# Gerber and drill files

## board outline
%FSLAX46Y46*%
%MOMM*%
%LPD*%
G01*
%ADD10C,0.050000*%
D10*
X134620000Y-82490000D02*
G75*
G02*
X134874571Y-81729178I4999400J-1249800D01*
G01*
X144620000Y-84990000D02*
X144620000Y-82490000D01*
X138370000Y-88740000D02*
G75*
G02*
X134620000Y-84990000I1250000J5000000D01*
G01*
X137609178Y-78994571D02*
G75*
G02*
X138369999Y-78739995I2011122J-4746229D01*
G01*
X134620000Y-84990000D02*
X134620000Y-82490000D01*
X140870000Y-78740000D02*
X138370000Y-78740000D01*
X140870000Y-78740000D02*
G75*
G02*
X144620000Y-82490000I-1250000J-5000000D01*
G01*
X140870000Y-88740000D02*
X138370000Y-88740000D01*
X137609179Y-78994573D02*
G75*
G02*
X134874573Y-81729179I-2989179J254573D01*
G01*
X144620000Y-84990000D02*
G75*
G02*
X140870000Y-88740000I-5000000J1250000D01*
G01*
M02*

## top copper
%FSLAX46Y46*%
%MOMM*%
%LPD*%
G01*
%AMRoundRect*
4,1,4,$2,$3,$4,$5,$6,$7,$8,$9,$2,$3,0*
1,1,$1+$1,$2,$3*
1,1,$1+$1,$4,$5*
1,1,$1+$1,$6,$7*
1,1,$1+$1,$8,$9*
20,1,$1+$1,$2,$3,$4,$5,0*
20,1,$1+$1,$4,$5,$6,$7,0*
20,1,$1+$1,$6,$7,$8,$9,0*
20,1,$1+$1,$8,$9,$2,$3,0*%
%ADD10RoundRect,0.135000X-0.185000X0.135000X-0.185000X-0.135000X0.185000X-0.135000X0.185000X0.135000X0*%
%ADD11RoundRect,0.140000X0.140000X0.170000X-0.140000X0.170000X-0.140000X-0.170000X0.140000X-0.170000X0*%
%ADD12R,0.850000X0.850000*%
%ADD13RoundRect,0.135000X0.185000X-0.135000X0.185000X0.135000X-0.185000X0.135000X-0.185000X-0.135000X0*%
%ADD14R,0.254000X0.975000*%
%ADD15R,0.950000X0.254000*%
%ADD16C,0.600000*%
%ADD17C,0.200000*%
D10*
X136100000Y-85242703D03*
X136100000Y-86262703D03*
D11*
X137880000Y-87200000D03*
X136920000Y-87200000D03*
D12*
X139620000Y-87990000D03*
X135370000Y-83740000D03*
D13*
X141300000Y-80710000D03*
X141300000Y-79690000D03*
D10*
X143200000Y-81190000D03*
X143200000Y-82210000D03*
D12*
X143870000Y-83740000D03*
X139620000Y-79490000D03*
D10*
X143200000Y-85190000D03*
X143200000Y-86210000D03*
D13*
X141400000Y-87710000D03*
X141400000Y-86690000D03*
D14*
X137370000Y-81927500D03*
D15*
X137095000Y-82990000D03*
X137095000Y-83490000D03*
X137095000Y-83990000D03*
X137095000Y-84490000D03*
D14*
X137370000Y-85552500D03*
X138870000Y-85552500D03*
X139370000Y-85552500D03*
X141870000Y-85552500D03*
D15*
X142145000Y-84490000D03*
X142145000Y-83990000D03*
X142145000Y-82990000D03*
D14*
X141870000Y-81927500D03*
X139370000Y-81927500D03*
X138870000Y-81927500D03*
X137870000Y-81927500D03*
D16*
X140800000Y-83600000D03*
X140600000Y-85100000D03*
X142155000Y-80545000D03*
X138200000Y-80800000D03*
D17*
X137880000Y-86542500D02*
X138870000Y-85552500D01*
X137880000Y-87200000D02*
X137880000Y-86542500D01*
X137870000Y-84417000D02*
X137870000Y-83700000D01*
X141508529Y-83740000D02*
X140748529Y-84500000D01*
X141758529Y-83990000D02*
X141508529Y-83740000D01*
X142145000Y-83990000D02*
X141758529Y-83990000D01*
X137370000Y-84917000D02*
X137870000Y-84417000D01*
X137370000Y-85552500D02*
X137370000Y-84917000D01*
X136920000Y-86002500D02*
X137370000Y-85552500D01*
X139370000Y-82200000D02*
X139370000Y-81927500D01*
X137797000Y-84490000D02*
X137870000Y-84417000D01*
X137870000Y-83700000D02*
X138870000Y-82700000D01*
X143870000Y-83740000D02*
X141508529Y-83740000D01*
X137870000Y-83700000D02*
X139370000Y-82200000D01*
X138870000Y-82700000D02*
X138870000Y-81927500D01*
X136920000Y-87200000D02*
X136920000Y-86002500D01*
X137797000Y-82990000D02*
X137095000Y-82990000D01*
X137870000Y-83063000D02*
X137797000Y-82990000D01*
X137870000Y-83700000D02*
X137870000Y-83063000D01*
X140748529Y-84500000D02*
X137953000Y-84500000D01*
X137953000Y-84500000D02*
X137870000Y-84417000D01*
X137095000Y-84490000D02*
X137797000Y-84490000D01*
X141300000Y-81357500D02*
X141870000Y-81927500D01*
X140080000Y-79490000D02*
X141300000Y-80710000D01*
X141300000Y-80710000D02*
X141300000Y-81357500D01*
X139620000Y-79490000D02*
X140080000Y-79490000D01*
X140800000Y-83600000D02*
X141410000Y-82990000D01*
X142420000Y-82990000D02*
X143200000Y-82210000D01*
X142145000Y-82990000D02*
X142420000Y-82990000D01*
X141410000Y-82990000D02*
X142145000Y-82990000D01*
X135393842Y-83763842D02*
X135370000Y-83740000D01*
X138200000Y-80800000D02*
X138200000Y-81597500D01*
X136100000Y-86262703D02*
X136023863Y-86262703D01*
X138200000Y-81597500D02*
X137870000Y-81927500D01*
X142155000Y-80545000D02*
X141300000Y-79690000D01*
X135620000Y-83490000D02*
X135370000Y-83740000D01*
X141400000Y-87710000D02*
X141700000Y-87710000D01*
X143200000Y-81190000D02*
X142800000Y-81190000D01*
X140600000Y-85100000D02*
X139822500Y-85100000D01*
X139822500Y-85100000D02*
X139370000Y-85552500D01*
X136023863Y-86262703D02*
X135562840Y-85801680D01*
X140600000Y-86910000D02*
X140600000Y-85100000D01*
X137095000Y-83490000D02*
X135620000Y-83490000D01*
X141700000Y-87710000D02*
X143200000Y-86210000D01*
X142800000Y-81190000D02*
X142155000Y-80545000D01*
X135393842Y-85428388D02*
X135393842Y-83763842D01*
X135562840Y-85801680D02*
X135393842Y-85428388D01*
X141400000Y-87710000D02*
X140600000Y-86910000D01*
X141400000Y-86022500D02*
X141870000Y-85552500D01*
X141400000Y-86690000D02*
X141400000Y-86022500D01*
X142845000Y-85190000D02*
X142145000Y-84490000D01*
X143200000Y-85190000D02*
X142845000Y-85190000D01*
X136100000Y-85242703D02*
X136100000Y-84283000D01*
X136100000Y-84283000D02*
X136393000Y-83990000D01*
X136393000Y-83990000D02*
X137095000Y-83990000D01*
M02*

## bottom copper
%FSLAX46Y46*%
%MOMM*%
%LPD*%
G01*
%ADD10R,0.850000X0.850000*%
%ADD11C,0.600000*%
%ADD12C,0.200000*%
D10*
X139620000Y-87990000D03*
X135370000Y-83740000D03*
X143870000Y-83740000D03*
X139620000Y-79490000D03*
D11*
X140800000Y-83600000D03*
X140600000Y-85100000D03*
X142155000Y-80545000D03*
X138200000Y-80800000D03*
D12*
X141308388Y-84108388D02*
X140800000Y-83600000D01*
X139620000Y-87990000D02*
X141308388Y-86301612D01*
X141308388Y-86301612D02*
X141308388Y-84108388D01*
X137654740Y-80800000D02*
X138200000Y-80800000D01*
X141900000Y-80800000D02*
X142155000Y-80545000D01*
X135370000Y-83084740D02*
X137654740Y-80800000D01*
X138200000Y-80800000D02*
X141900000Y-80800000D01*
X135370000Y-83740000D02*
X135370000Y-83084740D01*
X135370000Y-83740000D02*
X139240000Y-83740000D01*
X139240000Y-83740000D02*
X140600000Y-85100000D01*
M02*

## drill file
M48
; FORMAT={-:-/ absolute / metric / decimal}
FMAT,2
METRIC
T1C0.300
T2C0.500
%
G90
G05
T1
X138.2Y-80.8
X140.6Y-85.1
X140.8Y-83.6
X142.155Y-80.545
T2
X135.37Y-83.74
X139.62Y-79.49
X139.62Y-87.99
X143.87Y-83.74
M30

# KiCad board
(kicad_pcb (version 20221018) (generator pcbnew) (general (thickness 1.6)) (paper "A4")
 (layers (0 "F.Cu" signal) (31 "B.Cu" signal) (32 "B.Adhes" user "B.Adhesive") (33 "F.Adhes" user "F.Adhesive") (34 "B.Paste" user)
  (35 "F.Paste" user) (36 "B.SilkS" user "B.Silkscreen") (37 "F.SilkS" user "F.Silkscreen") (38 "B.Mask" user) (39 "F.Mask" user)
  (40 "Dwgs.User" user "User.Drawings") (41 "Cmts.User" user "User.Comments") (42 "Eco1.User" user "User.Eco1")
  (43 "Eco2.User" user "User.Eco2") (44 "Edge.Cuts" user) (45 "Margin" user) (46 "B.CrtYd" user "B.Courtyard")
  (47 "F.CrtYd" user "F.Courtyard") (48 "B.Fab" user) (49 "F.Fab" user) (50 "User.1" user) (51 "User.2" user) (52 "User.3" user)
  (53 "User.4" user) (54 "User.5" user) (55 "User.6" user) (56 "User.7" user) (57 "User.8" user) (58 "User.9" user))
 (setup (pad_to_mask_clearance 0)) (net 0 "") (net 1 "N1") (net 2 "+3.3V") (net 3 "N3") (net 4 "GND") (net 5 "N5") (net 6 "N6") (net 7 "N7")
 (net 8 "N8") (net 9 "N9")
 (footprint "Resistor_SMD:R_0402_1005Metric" (layer "F.Cu") (at 136.1 85.752703 -90)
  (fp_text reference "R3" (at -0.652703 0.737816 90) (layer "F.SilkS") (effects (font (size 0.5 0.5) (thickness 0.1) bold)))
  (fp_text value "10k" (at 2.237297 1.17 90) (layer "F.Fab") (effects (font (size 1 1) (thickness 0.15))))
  (pad "1" smd roundrect (at -0.51 0 270) (size 0.54 0.64) (layers "F.Cu" "F.Paste" "F.Mask") (roundrect_rratio 0.25) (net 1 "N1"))
  (pad "2" smd roundrect (at 0.51 0 270) (size 0.54 0.64) (layers "F.Cu" "F.Paste" "F.Mask") (roundrect_rratio 0.25) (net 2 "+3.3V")))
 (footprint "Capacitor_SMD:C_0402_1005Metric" (layer "F.Cu") (at 137.4 87.2 180)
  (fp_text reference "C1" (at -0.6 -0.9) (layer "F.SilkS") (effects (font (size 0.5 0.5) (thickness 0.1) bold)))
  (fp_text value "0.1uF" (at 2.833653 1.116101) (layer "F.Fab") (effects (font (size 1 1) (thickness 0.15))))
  (pad "1" smd roundrect (at -0.48 0 180) (size 0.56 0.62) (layers "F.Cu" "F.Paste" "F.Mask") (roundrect_rratio 0.25) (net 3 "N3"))
  (pad "2" smd roundrect (at 0.48 0 180) (size 0.56 0.62) (layers "F.Cu" "F.Paste" "F.Mask") (roundrect_rratio 0.25) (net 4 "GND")))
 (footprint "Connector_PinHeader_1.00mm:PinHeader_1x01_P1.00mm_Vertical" (layer "F.Cu") (at 139.62 87.99)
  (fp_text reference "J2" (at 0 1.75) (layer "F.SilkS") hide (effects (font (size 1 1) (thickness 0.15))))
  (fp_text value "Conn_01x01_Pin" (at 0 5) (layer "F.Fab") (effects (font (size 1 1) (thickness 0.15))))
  (pad "1" thru_hole rect (at 0 0) (size 0.85 0.85) (drill 0.5) (layers "*.Cu" "*.Mask") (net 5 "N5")))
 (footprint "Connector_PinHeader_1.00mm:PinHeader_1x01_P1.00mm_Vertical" (layer "F.Cu") (at 135.37 83.74)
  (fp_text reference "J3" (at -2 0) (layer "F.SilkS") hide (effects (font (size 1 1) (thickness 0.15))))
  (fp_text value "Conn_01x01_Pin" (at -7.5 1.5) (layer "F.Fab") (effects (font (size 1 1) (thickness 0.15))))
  (pad "1" thru_hole rect (at 0 0) (size 0.85 0.85) (drill 0.5) (layers "*.Cu" "*.Mask") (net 2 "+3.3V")))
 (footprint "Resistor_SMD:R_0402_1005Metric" (layer "F.Cu") (at 141.3 80.2 90)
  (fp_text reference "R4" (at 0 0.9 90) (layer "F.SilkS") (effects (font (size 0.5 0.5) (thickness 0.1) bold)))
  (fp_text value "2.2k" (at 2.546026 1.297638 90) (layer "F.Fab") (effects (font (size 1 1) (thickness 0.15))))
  (pad "1" smd roundrect (at -0.51 0 90) (size 0.54 0.64) (layers "F.Cu" "F.Paste" "F.Mask") (roundrect_rratio 0.25) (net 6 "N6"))
  (pad "2" smd roundrect (at 0.51 0 90) (size 0.54 0.64) (layers "F.Cu" "F.Paste" "F.Mask") (roundrect_rratio 0.25) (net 2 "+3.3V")))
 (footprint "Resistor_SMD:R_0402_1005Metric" (layer "F.Cu") (at 143.2 81.7 -90)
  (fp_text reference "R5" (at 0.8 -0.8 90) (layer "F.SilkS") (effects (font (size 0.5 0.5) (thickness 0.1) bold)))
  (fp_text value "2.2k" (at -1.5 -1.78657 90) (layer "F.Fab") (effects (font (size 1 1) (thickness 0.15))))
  (pad "1" smd roundrect (at -0.51 0 270) (size 0.54 0.64) (layers "F.Cu" "F.Paste" "F.Mask") (roundrect_rratio 0.25) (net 2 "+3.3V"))
  (pad "2" smd roundrect (at 0.51 0 270) (size 0.54 0.64) (layers "F.Cu" "F.Paste" "F.Mask") (roundrect_rratio 0.25) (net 5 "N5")))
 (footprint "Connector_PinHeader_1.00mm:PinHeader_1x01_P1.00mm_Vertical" (layer "F.Cu") (at 143.87 83.74)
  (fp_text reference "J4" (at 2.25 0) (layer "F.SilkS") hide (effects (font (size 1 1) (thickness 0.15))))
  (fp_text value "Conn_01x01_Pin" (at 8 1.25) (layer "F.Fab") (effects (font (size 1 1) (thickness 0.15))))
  (pad "1" thru_hole rect (at 0 0) (size 0.85 0.85) (drill 0.5) (layers "*.Cu" "*.Mask") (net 4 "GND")))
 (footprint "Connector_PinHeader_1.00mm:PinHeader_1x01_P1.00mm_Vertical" (layer "F.Cu") (at 139.62 79.49)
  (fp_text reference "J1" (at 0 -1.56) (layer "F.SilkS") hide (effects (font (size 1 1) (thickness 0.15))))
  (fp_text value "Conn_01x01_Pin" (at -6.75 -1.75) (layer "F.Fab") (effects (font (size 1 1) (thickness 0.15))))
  (pad "1" thru_hole rect (at 0 0) (size 0.85 0.85) (drill 0.5) (layers "*.Cu" "*.Mask") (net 6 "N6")))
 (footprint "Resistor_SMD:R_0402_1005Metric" (layer "F.Cu") (at 143.2 85.7 -90)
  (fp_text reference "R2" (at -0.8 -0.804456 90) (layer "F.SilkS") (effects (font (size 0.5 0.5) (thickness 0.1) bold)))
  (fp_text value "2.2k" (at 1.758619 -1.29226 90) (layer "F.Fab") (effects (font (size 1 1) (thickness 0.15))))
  (pad "1" smd roundrect (at -0.51 0 270) (size 0.54 0.64) (layers "F.Cu" "F.Paste" "F.Mask") (roundrect_rratio 0.25) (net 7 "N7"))
  (pad "2" smd roundrect (at 0.51 0 270) (size 0.54 0.64) (layers "F.Cu" "F.Paste" "F.Mask") (roundrect_rratio 0.25) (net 2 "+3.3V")))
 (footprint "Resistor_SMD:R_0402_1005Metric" (layer "F.Cu") (at 141.4 87.2 90)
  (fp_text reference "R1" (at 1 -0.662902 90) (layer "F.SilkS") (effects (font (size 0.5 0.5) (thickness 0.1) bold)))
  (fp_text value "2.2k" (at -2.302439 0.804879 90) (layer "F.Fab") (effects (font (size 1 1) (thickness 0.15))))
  (pad "1" smd roundrect (at -0.51 0 90) (size 0.54 0.64) (layers "F.Cu" "F.Paste" "F.Mask") (roundrect_rratio 0.25) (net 2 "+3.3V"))
  (pad "2" smd roundrect (at 0.51 0 90) (size 0.54 0.64) (layers "F.Cu" "F.Paste" "F.Mask") (roundrect_rratio 0.25) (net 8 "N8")))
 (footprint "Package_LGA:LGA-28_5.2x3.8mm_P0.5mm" (layer "F.Cu") (at 139.62 83.74)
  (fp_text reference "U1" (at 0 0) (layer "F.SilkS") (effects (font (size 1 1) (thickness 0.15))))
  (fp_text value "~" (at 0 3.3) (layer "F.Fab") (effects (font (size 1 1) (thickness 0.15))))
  (pad "1" smd rect (at -2.25 -1.8125) (size 0.254 0.975) (layers "F.Cu" "F.Paste" "F.Mask") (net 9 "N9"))
  (pad "2" smd rect (at -2.525 -0.75 90) (size 0.254 0.95) (layers "F.Cu" "F.Paste" "F.Mask") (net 4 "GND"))
  (pad "3" smd rect (at -2.525 -0.25 90) (size 0.254 0.95) (layers "F.Cu" "F.Paste" "F.Mask") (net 2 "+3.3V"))
  (pad "4" smd rect (at -2.525 0.25 90) (size 0.254 0.95) (layers "F.Cu" "F.Paste" "F.Mask") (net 1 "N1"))
  (pad "5" smd rect (at -2.525 0.75 90) (size 0.254 0.95) (layers "F.Cu" "F.Paste" "F.Mask") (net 4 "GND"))
  (pad "6" smd rect (at -2.25 1.8125) (size 0.254 0.975) (layers "F.Cu" "F.Paste" "F.Mask") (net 4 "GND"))
  (pad "9" smd rect (at -0.75 1.8125) (size 0.254 0.975) (layers "F.Cu" "F.Paste" "F.Mask") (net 3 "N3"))
  (pad "10" smd rect (at -0.25 1.8125) (size 0.254 0.975) (layers "F.Cu" "F.Paste" "F.Mask") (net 2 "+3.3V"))
  (pad "15" smd rect (at 2.25 1.8125) (size 0.254 0.975) (layers "F.Cu" "F.Paste" "F.Mask") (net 8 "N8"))
  (pad "16" smd rect (at 2.525 0.75 90) (size 0.254 0.95) (layers "F.Cu" "F.Paste" "F.Mask") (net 7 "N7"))
  (pad "17" smd rect (at 2.525 0.25 90) (size 0.254 0.95) (layers "F.Cu" "F.Paste" "F.Mask") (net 4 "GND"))
  (pad "19" smd rect (at 2.525 -0.75 90) (size 0.254 0.95) (layers "F.Cu" "F.Paste" "F.Mask") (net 5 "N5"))
  (pad "20" smd rect (at 2.25 -1.8125) (size 0.254 0.975) (layers "F.Cu" "F.Paste" "F.Mask") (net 6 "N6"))
  (pad "25" smd rect (at -0.25 -1.8125) (size 0.254 0.975) (layers "F.Cu" "F.Paste" "F.Mask") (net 4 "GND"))
  (pad "26" smd rect (at -0.75 -1.8125) (size 0.254 0.975) (layers "F.Cu" "F.Paste" "F.Mask") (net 4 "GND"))
  (pad "28" smd rect (at -1.75 -1.8125) (size 0.254 0.975) (layers "F.Cu" "F.Paste" "F.Mask") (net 2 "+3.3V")))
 (gr_arc (start 134.62 82.49) (mid 134.732457 82.104627) (end 134.874571 81.729178) (stroke (width 0.05) (type default)) (layer "Edge.Cuts"))
 (gr_line (start 144.62 84.99) (end 144.62 82.49) (stroke (width 0.05) (type default)) (layer "Edge.Cuts"))
 (gr_arc (start 138.37 88.74) (mid 135.975655 87.384345) (end 134.62 84.99) (stroke (width 0.05) (type default)) (layer "Edge.Cuts"))
 (gr_arc (start 137.609178 78.994571) (mid 137.984629 78.852461) (end 138.37 78.74) (stroke (width 0.05) (type default)) (layer "Edge.Cuts"))
 (gr_line (start 134.62 84.99) (end 134.62 82.49) (stroke (width 0.05) (type default)) (layer "Edge.Cuts"))
 (gr_line (start 140.87 78.74) (end 138.37 78.74) (stroke (width 0.05) (type default)) (layer "Edge.Cuts"))
 (gr_arc (start 140.87 78.74) (mid 143.264345 80.095655) (end 144.62 82.49) (stroke (width 0.05) (type default)) (layer "Edge.Cuts"))
 (gr_line (start 140.87 88.74) (end 138.37 88.74) (stroke (width 0.05) (type default)) (layer "Edge.Cuts"))
 (gr_arc (start 137.609179 78.994573) (mid 136.74132 80.86132) (end 134.874573 81.729179) (stroke (width 0.05) (type default))
  (layer "Edge.Cuts"))
 (gr_arc (start 144.62 84.99) (mid 143.264345 87.384345) (end 140.87 88.74) (stroke (width 0.05) (type default)) (layer "Edge.Cuts"))
 (segment (start 137.88 86.5425) (end 138.87 85.5525) (width 0.2) (layer "F.Cu") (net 3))
 (segment (start 137.88 87.2) (end 137.88 86.5425) (width 0.2) (layer "F.Cu") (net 3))
 (segment (start 137.87 84.417) (end 137.87 83.7) (width 0.2) (layer "F.Cu") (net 4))
 (segment (start 141.508529 83.74) (end 140.748529 84.5) (width 0.2) (layer "F.Cu") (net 4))
 (segment (start 141.758529 83.99) (end 141.508529 83.74) (width 0.2) (layer "F.Cu") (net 4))
 (segment (start 142.145 83.99) (end 141.758529 83.99) (width 0.2) (layer "F.Cu") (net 4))
 (segment (start 137.37 84.917) (end 137.87 84.417) (width 0.2) (layer "F.Cu") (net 4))
 (segment (start 137.37 85.5525) (end 137.37 84.917) (width 0.2) (layer "F.Cu") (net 4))
 (segment (start 136.92 86.0025) (end 137.37 85.5525) (width 0.2) (layer "F.Cu") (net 4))
 (segment (start 139.37 82.2) (end 139.37 81.9275) (width 0.2) (layer "F.Cu") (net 4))
 (segment (start 137.797 84.49) (end 137.87 84.417) (width 0.2) (layer "F.Cu") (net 4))
 (segment (start 137.87 83.7) (end 138.87 82.7) (width 0.2) (layer "F.Cu") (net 4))
 (segment (start 143.87 83.74) (end 141.508529 83.74) (width 0.2) (layer "F.Cu") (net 4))
 (segment (start 137.87 83.7) (end 139.37 82.2) (width 0.2) (layer "F.Cu") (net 4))
 (segment (start 138.87 82.7) (end 138.87 81.9275) (width 0.2) (layer "F.Cu") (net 4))
 (segment (start 136.92 87.2) (end 136.92 86.0025) (width 0.2) (layer "F.Cu") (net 4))
 (segment (start 137.797 82.99) (end 137.095 82.99) (width 0.2) (layer "F.Cu") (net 4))
 (segment (start 137.87 83.063) (end 137.797 82.99) (width 0.2) (layer "F.Cu") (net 4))
 (segment (start 137.87 83.7) (end 137.87 83.063) (width 0.2) (layer "F.Cu") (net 4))
 (segment (start 140.748529 84.5) (end 137.953 84.5) (width 0.2) (layer "F.Cu") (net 4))
 (segment (start 137.953 84.5) (end 137.87 84.417) (width 0.2) (layer "F.Cu") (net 4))
 (segment (start 137.095 84.49) (end 137.797 84.49) (width 0.2) (layer "F.Cu") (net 4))
 (segment (start 141.3 81.3575) (end 141.87 81.9275) (width 0.2) (layer "F.Cu") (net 6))
 (segment (start 140.08 79.49) (end 141.3 80.71) (width 0.2) (layer "F.Cu") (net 6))
 (segment (start 141.3 80.71) (end 141.3 81.3575) (width 0.2) (layer "F.Cu") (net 6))
 (segment (start 139.62 79.49) (end 140.08 79.49) (width 0.2) (layer "F.Cu") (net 6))
 (segment (start 140.8 83.6) (end 141.41 82.99) (width 0.2) (layer "F.Cu") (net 5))
 (segment (start 142.42 82.99) (end 143.2 82.21) (width 0.2) (layer "F.Cu") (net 5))
 (segment (start 142.145 82.99) (end 142.42 82.99) (width 0.2) (layer "F.Cu") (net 5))
 (segment (start 141.41 82.99) (end 142.145 82.99) (width 0.2) (layer "F.Cu") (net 5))
 (via (at 140.8 83.6) (size 0.6) (drill 0.3) (layers "F.Cu" "B.Cu") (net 5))
 (segment (start 141.308388 84.108388) (end 140.8 83.6) (width 0.2) (layer "B.Cu") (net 5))
 (segment (start 139.62 87.99) (end 141.308388 86.301612) (width 0.2) (layer "B.Cu") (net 5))
 (segment (start 141.308388 86.301612) (end 141.308388 84.108388) (width 0.2) (layer "B.Cu") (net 5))
 (segment (start 135.393842 83.763842) (end 135.37 83.74) (width 0.2) (layer "F.Cu") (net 2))
 (segment (start 138.2 80.8) (end 138.2 81.5975) (width 0.2) (layer "F.Cu") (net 2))
 (segment (start 136.1 86.262703) (end 136.023863 86.262703) (width 0.2) (layer "F.Cu") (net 2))
 (segment (start 138.2 81.5975) (end 137.87 81.9275) (width 0.2) (layer "F.Cu") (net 2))
 (segment (start 142.155 80.545) (end 141.3 79.69) (width 0.2) (layer "F.Cu") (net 2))
 (segment (start 135.62 83.49) (end 135.37 83.74) (width 0.2) (layer "F.Cu") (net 2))
 (segment (start 141.4 87.71) (end 141.7 87.71) (width 0.2) (layer "F.Cu") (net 2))
 (segment (start 143.2 81.19) (end 142.8 81.19) (width 0.2) (layer "F.Cu") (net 2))
 (segment (start 140.6 85.1) (end 139.8225 85.1) (width 0.2) (layer "F.Cu") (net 2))
 (segment (start 139.8225 85.1) (end 139.37 85.5525) (width 0.2) (layer "F.Cu") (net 2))
 (segment (start 136.023863 86.262703) (end 135.56284 85.80168) (width 0.2) (layer "F.Cu") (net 2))
 (segment (start 140.6 86.91) (end 140.6 85.1) (width 0.2) (layer "F.Cu") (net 2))
 (segment (start 137.095 83.49) (end 135.62 83.49) (width 0.2) (layer "F.Cu") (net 2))
 (segment (start 141.7 87.71) (end 143.2 86.21) (width 0.2) (layer "F.Cu") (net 2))
 (segment (start 142.8 81.19) (end 142.155 80.545) (width 0.2) (layer "F.Cu") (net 2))
 (segment (start 135.393842 85.428388) (end 135.393842 83.763842) (width 0.2) (layer "F.Cu") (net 2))
 (segment (start 135.56284 85.80168) (end 135.393842 85.428388) (width 0.2) (layer "F.Cu") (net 2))
 (segment (start 141.4 87.71) (end 140.6 86.91) (width 0.2) (layer "F.Cu") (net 2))
 (via (at 140.6 85.1) (size 0.6) (drill 0.3) (layers "F.Cu" "B.Cu") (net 2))
 (via (at 142.155 80.545) (size 0.6) (drill 0.3) (layers "F.Cu" "B.Cu") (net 2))
 (via (at 138.2 80.8) (size 0.6) (drill 0.3) (layers "F.Cu" "B.Cu") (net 2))
 (segment (start 137.65474 80.8) (end 138.2 80.8) (width 0.2) (layer "B.Cu") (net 2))
 (segment (start 141.9 80.8) (end 142.155 80.545) (width 0.2) (layer "B.Cu") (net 2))
 (segment (start 135.37 83.08474) (end 137.65474 80.8) (width 0.2) (layer "B.Cu") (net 2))
 (segment (start 138.2 80.8) (end 141.9 80.8) (width 0.2) (layer "B.Cu") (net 2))
 (segment (start 135.37 83.74) (end 135.37 83.08474) (width 0.2) (layer "B.Cu") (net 2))
 (segment (start 135.37 83.74) (end 139.24 83.74) (width 0.2) (layer "B.Cu") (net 2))
 (segment (start 139.24 83.74) (end 140.6 85.1) (width 0.2) (layer "B.Cu") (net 2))
 (segment (start 141.4 86.0225) (end 141.87 85.5525) (width 0.2) (layer "F.Cu") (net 8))
 (segment (start 141.4 86.69) (end 141.4 86.0225) (width 0.2) (layer "F.Cu") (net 8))
 (segment (start 142.845 85.19) (end 142.145 84.49) (width 0.2) (layer "F.Cu") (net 7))
 (segment (start 143.2 85.19) (end 142.845 85.19) (width 0.2) (layer "F.Cu") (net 7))
 (segment (start 136.1 85.242703) (end 136.1 84.283) (width 0.2) (layer "F.Cu") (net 1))
 (segment (start 136.1 84.283) (end 136.393 83.99) (width 0.2) (layer "F.Cu") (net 1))
 (segment (start 136.393 83.99) (end 137.095 83.99) (width 0.2) (layer "F.Cu") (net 1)))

